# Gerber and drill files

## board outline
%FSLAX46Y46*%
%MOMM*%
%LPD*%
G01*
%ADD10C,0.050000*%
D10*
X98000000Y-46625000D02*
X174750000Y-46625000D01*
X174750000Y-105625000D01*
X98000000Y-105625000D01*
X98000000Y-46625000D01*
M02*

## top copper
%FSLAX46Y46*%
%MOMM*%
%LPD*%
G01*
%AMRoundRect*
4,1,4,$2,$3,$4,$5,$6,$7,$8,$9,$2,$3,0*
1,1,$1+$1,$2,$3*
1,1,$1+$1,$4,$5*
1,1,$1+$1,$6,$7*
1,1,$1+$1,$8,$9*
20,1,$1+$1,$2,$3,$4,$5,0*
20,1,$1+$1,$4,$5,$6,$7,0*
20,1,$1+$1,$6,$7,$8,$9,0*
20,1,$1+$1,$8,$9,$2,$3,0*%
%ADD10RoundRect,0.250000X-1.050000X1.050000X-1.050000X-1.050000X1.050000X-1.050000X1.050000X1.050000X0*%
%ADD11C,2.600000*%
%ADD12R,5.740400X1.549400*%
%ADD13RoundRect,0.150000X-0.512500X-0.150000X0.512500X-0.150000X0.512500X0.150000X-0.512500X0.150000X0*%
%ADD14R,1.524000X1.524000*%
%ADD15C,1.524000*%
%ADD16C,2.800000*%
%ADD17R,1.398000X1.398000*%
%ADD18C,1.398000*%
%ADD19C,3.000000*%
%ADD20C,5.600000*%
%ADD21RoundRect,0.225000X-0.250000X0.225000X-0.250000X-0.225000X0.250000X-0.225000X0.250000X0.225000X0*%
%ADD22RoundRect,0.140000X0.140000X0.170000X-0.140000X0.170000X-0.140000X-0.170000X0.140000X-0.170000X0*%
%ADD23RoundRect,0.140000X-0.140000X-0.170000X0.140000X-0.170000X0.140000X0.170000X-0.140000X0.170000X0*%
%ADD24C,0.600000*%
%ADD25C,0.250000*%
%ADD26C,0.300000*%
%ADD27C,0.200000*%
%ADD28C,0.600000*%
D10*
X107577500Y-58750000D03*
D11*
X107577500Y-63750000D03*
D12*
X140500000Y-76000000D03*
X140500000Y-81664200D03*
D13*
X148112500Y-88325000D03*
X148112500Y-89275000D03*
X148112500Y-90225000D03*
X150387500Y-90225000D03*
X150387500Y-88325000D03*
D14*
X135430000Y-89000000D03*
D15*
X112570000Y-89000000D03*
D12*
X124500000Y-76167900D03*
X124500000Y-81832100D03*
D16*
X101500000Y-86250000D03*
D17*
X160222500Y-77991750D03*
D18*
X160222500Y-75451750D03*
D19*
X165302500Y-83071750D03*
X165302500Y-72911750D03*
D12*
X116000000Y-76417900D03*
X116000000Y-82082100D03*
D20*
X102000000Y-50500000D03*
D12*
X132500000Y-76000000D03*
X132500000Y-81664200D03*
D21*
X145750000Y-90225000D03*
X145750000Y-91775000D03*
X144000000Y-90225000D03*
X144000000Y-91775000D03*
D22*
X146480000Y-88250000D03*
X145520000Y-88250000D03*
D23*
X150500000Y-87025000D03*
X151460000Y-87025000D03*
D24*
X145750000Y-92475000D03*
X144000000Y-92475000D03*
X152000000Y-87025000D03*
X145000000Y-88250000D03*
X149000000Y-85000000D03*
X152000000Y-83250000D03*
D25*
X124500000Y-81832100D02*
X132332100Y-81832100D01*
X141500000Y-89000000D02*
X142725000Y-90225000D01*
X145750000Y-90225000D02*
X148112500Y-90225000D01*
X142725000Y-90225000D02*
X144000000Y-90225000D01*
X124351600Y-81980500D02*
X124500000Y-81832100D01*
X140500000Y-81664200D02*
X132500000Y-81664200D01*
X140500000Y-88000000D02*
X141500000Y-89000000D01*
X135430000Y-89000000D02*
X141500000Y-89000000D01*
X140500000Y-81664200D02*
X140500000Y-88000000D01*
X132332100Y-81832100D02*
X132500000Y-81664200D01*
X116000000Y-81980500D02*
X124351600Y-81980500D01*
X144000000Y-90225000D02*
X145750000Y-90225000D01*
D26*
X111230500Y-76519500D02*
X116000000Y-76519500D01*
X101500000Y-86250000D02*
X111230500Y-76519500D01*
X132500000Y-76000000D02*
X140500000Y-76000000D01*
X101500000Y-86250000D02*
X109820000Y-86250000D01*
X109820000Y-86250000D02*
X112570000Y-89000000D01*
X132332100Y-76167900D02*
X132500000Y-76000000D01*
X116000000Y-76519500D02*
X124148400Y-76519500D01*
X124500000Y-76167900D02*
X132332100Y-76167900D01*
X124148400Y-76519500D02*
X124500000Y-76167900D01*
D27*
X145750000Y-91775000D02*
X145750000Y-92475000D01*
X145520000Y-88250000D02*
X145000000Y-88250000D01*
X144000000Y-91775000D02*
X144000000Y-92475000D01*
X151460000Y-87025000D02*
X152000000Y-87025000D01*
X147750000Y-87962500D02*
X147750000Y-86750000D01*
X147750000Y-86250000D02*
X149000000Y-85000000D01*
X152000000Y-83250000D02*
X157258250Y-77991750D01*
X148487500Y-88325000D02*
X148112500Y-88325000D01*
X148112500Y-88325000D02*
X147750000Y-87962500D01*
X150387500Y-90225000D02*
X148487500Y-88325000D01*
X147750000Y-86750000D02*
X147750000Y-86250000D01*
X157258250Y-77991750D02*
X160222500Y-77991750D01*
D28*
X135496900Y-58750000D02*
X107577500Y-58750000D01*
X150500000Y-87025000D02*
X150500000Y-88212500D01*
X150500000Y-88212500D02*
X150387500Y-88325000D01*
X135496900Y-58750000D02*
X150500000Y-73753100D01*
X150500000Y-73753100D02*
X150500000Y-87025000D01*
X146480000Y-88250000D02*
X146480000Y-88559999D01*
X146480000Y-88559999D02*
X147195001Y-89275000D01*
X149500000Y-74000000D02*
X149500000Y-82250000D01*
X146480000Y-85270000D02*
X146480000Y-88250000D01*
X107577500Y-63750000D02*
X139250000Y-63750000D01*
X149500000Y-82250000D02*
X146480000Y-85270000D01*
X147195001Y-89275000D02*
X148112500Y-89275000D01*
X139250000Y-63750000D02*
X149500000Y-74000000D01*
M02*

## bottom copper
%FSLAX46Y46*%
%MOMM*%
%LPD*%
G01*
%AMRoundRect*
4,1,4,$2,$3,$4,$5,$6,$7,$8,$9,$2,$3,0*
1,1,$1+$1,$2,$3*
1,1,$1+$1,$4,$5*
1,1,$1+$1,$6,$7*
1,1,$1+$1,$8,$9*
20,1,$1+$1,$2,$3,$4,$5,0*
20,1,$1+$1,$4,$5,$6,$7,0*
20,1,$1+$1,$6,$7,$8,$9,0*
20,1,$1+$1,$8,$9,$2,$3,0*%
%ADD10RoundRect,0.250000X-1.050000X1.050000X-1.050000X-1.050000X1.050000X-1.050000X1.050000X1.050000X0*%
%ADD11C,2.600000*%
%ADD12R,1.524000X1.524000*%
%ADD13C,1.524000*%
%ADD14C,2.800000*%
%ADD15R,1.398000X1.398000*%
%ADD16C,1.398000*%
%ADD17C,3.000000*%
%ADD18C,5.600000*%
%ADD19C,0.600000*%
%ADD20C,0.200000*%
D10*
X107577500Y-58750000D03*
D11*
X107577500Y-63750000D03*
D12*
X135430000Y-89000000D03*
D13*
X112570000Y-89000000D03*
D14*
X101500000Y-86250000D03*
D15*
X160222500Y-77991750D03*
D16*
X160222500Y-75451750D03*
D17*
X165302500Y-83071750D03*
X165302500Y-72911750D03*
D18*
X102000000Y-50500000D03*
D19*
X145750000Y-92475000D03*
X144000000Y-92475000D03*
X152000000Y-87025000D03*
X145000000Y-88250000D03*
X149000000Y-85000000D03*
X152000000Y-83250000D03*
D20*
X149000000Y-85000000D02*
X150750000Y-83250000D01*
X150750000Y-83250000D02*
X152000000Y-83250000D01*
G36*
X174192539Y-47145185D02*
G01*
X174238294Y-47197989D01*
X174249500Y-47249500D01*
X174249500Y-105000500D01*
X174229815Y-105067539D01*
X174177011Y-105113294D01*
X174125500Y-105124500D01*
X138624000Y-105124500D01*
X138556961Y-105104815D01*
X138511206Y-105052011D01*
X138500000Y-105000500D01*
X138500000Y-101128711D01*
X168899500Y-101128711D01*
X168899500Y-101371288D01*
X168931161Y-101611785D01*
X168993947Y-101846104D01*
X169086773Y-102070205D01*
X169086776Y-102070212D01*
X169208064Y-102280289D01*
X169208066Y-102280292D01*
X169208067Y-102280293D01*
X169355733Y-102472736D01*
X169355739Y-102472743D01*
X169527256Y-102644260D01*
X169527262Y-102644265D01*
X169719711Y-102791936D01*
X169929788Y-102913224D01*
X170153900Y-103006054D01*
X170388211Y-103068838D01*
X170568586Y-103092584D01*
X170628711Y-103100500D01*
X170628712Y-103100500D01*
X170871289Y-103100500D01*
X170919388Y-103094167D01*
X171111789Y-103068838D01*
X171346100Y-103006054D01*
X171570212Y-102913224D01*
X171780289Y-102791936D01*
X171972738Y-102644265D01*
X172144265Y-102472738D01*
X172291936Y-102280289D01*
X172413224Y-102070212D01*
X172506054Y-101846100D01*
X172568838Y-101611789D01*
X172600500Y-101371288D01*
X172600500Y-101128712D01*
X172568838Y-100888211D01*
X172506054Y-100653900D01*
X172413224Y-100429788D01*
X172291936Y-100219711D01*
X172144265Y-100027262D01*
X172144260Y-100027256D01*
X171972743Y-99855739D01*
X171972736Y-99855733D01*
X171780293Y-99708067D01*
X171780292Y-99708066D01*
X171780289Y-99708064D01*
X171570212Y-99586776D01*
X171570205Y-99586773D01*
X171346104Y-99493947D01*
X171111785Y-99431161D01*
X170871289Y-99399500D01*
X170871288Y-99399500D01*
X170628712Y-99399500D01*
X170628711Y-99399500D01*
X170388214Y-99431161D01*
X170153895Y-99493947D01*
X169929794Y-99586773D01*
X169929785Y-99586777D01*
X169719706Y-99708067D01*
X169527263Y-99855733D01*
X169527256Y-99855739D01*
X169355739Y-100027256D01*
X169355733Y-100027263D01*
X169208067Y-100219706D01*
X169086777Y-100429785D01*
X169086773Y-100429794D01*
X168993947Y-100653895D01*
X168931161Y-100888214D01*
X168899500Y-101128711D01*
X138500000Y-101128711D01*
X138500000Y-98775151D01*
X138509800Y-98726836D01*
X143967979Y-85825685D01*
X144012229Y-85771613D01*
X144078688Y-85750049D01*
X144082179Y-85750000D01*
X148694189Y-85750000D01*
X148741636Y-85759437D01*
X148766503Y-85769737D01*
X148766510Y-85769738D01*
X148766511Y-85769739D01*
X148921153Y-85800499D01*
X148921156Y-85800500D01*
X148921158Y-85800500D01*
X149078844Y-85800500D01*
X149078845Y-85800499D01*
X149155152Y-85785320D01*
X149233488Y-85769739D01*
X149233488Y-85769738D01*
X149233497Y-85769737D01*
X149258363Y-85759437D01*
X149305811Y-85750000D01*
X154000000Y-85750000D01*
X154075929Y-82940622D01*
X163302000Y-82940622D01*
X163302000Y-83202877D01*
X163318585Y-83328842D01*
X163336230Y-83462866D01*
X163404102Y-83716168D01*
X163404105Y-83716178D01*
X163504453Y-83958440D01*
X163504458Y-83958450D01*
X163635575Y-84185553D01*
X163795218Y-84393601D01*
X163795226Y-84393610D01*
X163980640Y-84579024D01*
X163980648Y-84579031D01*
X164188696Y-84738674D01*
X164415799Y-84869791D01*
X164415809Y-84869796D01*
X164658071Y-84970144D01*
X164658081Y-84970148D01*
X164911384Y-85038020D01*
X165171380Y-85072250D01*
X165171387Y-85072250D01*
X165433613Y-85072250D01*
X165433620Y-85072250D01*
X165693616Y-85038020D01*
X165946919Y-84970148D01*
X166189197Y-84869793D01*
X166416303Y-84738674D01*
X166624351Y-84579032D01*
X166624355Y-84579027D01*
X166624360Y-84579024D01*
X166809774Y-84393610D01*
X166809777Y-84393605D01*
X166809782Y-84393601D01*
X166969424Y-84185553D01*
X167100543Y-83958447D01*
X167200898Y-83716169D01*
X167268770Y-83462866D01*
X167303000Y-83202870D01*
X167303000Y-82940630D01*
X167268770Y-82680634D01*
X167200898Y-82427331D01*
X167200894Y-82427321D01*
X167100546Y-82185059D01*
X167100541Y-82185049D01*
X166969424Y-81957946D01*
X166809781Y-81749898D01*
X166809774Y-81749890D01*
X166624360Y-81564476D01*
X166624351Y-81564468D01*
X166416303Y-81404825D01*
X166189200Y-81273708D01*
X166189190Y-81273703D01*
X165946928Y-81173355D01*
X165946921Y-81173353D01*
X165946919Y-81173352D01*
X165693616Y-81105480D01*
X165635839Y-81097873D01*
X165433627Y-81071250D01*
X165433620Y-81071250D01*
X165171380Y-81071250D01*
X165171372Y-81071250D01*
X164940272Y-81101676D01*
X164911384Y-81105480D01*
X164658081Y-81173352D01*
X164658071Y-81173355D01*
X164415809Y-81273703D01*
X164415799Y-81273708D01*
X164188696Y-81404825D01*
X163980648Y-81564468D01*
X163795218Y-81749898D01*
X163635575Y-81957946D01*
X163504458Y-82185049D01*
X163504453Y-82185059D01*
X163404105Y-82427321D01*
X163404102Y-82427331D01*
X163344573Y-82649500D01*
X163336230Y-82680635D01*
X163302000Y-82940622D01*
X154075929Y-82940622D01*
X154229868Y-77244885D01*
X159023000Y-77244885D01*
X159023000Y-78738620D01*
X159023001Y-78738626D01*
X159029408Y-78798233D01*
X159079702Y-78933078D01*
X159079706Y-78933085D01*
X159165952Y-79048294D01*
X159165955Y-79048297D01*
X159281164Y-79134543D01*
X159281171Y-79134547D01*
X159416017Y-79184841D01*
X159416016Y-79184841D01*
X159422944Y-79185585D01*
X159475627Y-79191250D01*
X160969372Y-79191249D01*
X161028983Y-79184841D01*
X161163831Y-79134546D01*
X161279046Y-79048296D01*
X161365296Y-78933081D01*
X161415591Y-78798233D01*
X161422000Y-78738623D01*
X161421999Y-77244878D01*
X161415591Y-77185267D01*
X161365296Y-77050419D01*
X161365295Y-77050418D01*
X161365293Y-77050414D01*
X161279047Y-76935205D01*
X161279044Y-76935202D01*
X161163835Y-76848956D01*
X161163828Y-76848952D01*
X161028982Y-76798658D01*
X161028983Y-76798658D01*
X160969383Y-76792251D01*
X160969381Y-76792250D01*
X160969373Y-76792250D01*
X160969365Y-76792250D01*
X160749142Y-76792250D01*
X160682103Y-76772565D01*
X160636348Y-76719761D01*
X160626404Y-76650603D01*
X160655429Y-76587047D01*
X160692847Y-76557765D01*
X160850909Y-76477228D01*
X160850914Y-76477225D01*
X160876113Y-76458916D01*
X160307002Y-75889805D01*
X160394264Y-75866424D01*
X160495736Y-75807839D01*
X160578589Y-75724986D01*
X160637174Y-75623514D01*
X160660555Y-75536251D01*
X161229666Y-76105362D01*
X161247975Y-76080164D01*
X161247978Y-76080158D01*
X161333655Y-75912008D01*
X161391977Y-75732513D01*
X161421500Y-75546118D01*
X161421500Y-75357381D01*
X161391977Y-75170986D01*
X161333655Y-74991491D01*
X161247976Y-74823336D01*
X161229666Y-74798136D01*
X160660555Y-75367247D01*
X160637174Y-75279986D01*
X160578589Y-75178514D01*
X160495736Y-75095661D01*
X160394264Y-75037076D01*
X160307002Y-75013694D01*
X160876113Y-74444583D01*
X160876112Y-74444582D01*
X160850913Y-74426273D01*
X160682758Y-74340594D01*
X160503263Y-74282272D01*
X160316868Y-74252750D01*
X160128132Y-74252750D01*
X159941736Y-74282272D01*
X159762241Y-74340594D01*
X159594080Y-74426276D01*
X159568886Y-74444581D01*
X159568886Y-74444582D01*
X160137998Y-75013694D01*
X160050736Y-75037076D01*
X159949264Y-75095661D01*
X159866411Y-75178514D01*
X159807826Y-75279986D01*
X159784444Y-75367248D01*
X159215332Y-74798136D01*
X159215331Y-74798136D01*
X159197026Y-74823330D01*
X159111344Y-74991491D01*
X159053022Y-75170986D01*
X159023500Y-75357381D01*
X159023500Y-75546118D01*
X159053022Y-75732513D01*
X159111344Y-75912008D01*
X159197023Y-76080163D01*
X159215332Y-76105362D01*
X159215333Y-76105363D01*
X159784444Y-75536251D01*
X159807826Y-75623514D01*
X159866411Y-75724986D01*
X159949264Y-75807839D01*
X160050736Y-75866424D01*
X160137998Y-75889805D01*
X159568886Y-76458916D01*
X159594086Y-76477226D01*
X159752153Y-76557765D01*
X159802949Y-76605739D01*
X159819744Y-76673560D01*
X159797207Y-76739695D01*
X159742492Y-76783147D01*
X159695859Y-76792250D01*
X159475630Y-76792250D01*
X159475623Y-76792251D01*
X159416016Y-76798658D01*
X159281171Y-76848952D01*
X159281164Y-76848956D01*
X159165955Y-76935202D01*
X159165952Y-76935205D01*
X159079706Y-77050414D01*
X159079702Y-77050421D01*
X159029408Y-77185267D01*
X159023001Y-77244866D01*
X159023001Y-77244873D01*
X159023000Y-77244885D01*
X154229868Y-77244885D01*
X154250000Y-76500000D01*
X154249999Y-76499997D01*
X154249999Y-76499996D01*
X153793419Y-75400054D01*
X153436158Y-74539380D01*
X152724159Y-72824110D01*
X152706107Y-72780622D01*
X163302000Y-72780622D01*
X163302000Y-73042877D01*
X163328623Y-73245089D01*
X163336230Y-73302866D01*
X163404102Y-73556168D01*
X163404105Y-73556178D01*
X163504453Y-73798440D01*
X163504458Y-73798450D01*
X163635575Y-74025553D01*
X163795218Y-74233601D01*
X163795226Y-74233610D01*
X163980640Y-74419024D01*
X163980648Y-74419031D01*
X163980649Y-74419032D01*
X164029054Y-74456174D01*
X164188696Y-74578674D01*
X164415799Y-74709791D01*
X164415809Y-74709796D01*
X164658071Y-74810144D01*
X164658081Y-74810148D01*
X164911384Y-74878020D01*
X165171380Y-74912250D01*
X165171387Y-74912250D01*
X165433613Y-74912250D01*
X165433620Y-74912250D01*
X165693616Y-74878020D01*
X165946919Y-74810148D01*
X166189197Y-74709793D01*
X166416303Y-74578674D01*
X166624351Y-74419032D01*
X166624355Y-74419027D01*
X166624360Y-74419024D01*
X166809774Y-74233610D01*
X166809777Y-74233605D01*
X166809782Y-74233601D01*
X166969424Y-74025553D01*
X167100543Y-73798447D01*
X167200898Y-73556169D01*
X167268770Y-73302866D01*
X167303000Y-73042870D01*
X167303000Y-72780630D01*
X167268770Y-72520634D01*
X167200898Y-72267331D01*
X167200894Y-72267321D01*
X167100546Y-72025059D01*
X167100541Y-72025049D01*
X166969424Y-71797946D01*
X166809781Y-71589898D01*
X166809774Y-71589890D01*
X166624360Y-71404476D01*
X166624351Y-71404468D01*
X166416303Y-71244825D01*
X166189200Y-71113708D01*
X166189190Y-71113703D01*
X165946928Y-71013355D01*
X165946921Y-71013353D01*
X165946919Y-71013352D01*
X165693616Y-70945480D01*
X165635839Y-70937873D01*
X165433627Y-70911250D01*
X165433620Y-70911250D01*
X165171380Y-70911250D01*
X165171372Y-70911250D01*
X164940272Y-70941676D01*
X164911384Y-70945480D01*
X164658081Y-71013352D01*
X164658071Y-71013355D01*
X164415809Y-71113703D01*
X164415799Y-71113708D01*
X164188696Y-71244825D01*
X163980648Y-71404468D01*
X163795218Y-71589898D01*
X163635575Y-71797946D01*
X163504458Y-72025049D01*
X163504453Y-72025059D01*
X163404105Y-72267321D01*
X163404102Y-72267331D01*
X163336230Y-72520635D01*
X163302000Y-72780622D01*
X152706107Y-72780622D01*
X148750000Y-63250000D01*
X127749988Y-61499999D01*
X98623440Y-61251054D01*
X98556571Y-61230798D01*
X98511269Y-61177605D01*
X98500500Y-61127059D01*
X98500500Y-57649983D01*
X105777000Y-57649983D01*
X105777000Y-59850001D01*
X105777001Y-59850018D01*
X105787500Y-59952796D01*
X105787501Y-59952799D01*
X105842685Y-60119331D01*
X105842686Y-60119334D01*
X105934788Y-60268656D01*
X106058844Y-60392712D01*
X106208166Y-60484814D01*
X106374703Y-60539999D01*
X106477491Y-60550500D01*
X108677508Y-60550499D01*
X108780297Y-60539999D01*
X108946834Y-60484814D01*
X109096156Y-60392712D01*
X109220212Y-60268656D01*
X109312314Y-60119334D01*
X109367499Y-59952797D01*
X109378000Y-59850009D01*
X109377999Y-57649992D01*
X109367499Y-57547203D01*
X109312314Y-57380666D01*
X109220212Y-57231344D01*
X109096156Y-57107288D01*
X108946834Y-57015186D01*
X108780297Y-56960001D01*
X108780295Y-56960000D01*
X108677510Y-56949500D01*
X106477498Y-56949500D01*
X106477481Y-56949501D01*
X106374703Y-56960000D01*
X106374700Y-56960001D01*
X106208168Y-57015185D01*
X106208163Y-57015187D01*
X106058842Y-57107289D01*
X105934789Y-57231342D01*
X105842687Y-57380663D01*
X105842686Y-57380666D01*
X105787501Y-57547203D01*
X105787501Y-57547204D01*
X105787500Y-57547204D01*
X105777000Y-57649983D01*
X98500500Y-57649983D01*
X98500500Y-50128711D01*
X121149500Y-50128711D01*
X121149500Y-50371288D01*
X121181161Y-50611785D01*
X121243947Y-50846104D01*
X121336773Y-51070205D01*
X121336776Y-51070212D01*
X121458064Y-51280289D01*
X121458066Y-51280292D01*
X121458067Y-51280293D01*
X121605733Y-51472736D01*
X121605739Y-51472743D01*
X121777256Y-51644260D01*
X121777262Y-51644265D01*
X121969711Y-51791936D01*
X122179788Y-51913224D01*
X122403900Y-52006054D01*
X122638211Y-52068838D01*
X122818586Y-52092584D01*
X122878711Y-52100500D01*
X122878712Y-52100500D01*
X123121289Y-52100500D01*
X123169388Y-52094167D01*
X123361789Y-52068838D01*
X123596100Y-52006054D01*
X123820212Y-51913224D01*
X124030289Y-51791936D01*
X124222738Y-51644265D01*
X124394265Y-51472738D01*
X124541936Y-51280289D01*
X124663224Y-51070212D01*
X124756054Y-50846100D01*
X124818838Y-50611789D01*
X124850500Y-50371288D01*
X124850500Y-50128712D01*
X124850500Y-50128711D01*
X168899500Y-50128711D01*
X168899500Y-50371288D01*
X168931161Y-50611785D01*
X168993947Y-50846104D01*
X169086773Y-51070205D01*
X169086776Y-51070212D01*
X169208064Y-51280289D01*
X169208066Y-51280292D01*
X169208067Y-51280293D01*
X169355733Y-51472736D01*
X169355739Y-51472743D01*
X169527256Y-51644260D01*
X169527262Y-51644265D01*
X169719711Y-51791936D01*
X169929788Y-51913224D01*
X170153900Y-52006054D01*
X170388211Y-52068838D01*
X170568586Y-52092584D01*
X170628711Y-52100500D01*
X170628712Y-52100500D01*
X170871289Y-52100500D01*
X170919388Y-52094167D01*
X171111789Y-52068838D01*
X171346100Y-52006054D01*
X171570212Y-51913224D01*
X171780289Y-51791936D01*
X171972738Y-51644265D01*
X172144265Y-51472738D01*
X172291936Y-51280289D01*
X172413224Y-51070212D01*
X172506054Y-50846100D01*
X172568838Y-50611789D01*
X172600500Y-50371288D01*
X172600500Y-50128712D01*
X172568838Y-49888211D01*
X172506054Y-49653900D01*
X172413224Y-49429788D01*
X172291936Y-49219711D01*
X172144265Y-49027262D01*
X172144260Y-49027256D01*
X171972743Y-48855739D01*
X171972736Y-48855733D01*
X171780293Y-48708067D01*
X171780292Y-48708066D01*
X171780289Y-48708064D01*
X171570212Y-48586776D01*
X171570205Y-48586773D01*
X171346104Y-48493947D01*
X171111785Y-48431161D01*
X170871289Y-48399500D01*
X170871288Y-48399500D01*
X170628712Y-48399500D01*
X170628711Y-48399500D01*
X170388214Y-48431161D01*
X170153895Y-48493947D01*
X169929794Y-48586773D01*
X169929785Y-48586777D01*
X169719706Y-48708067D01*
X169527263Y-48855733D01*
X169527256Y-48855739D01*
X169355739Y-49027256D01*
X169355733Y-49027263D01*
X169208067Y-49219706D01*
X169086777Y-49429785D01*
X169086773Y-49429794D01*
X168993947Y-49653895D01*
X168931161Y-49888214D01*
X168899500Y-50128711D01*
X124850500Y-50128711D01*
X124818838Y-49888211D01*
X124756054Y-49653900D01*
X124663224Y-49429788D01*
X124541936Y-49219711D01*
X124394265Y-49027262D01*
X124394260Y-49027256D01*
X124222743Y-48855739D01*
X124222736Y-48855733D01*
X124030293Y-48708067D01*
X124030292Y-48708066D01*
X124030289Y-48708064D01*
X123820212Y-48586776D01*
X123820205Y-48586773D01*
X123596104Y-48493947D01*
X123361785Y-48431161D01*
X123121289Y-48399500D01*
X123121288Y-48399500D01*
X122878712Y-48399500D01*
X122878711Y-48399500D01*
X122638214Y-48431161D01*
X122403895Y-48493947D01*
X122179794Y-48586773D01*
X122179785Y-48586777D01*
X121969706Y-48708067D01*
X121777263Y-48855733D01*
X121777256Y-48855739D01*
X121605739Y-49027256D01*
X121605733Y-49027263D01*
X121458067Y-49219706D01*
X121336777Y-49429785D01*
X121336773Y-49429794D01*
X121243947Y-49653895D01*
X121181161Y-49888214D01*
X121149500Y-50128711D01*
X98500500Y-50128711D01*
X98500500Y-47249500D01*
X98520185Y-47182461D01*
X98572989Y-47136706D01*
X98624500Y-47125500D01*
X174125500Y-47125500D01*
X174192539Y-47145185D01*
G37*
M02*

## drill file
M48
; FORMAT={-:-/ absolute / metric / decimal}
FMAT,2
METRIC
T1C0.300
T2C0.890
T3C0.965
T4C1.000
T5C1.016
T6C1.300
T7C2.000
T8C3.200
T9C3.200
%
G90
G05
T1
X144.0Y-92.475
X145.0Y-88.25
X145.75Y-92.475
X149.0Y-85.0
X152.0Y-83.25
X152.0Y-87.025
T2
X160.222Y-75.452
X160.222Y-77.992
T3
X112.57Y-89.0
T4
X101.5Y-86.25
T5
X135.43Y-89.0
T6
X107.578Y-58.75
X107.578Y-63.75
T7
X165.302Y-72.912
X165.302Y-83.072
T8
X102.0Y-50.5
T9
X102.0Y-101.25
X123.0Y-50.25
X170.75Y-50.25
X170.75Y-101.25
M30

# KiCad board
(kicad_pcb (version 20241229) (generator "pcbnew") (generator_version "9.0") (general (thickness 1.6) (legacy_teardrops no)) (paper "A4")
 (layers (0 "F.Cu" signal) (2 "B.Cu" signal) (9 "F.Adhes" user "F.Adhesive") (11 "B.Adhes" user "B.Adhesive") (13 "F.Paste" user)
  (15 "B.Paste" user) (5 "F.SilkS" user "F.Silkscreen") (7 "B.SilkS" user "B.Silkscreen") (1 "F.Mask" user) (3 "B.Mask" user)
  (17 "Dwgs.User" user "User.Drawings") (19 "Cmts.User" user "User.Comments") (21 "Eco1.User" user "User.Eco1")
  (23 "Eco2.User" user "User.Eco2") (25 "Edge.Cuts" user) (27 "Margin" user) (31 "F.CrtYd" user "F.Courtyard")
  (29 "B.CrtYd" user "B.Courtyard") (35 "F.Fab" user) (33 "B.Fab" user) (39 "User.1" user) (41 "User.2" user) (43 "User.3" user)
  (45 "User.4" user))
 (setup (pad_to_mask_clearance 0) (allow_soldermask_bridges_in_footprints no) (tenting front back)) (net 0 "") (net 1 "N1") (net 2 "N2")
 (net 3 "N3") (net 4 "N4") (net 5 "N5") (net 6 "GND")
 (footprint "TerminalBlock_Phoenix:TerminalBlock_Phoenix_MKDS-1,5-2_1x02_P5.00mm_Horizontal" (layer "F.Cu") (at 107.5775 58.75 -90)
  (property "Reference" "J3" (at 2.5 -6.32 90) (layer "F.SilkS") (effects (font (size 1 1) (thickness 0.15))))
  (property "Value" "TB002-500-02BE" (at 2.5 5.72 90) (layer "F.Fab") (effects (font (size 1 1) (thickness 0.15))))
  (pad "1" thru_hole roundrect (at 0 0 270) (size 2.6 2.6) (drill 1.3) (layers "*.Cu" "*.Mask") (remove_unused_layers no)
   (roundrect_rratio 0.096154) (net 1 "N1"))
  (pad "2" thru_hole circle (at 5 0 270) (size 2.6 2.6) (drill 1.3) (layers "*.Cu" "*.Mask") (remove_unused_layers no) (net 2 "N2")))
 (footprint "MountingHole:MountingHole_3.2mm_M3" (layer "F.Cu") (at 123 50.25)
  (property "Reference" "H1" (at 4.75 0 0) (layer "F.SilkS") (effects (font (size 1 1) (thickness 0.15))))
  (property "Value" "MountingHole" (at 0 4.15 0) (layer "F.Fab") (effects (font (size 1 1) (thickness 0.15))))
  (pad "" np_thru_hole circle (at 0 0) (size 3.2 3.2) (drill 3.2) (layers "*.Cu" "*.Mask")))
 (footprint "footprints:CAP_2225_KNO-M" (layer "F.Cu") (at 140.5 78.8321 -90)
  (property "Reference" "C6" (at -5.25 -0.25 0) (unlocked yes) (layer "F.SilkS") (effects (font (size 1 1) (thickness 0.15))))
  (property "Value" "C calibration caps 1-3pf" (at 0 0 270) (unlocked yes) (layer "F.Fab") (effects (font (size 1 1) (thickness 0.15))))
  (pad "1" smd rect (at -2.8321 0 270) (size 1.5494 5.7404) (layers "F.Cu" "F.Mask" "F.Paste") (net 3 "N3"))
  (pad "2" smd rect (at 2.8321 0 270) (size 1.5494 5.7404) (layers "F.Cu" "F.Mask" "F.Paste") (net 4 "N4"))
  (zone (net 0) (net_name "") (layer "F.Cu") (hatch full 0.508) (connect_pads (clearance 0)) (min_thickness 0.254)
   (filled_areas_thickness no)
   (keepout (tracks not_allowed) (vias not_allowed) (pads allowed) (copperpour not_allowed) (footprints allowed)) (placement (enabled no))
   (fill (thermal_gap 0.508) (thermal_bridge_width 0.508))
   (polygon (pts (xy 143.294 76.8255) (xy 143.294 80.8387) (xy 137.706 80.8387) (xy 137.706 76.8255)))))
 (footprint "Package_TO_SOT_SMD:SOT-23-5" (layer "F.Cu") (at 149.25 89.275)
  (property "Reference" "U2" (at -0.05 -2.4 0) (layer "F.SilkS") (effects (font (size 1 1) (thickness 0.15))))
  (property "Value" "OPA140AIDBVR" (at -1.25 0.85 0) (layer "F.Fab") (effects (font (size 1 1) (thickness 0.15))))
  (pad "1" smd roundrect (at -1.1375 -0.95) (size 1.325 0.6) (layers "F.Cu" "F.Mask" "F.Paste") (roundrect_rratio 0.25) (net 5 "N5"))
  (pad "2" smd roundrect (at -1.1375 0) (size 1.325 0.6) (layers "F.Cu" "F.Mask" "F.Paste") (roundrect_rratio 0.25) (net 2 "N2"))
  (pad "3" smd roundrect (at -1.1375 0.95) (size 1.325 0.6) (layers "F.Cu" "F.Mask" "F.Paste") (roundrect_rratio 0.25) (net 4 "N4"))
  (pad "4" smd roundrect (at 1.1375 0.95) (size 1.325 0.6) (layers "F.Cu" "F.Mask" "F.Paste") (roundrect_rratio 0.25) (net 5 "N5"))
  (pad "5" smd roundrect (at 1.1375 -0.95) (size 1.325 0.6) (layers "F.Cu" "F.Mask" "F.Paste") (roundrect_rratio 0.25) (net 1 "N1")))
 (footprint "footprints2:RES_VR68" (layer "F.Cu") (at 112.57 89 180)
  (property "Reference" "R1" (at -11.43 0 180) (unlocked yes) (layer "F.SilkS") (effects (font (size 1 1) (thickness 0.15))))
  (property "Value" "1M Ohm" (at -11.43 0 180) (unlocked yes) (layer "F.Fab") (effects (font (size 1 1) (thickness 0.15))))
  (pad "1" thru_hole rect (at -22.86 0 180) (size 1.524 1.524) (drill 1.016) (layers "*.Cu" "*.Mask") (remove_unused_layers no) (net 4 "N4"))
  (pad "2" thru_hole circle (at 0 0 180) (size 1.524 1.524) (drill 0.9652) (layers "*.Cu" "*.Mask") (remove_unused_layers no) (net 3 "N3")))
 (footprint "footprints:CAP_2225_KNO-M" (layer "F.Cu") (at 124.5 79 -90)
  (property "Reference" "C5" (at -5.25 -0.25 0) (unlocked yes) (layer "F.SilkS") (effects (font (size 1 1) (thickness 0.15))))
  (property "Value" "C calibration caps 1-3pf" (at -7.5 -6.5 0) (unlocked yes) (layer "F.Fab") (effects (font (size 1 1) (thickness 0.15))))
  (pad "1" smd rect (at -2.8321 0 270) (size 1.5494 5.7404) (layers "F.Cu" "F.Mask" "F.Paste") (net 3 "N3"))
  (pad "2" smd rect (at 2.8321 0 270) (size 1.5494 5.7404) (layers "F.Cu" "F.Mask" "F.Paste") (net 4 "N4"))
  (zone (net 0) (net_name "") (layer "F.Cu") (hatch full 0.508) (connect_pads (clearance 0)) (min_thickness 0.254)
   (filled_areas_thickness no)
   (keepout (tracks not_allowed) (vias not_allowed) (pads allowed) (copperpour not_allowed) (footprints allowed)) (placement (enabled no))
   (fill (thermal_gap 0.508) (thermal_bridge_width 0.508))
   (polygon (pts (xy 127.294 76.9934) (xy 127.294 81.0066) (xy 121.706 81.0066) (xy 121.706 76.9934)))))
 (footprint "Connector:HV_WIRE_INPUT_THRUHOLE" (layer "F.Cu") (at 101.5 89.25)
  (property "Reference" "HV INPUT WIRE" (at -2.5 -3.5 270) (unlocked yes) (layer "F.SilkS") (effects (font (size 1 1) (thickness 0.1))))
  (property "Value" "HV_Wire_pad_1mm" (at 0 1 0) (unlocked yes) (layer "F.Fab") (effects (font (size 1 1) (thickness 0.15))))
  (pad "1" thru_hole circle (at 0 -3) (size 2.8 2.8) (drill 1) (layers "*.Cu" "*.Mask") (remove_unused_layers no) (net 3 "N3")))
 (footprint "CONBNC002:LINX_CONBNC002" (layer "F.Cu") (at 165.3025 77.99175 90)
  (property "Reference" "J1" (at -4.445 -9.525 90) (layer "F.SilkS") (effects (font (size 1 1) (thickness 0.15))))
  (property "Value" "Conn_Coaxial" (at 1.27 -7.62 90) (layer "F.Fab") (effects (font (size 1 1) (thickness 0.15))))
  (pad "1" thru_hole rect (at 0 -5.08 90) (size 1.398 1.398) (drill 0.89) (layers "*.Cu" "*.Mask") (remove_unused_layers no) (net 5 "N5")
   (solder_mask_margin 0.102))
  (pad "2" thru_hole circle (at 2.54 -5.08 90) (size 1.398 1.398) (drill 0.89) (layers "*.Cu" "*.Mask") (remove_unused_layers no)
   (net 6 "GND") (solder_mask_margin 0.102))
  (pad "S1" thru_hole circle (at -5.08 0 90) (size 3 3) (drill 2) (layers "*.Cu" "*.Mask") (remove_unused_layers no)
   (solder_mask_margin 0.102))
  (pad "S2" thru_hole circle (at 5.08 0 90) (size 3 3) (drill 2) (layers "*.Cu" "*.Mask") (remove_unused_layers no)
   (solder_mask_margin 0.102)))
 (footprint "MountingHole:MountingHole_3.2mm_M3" (layer "F.Cu") (at 170.75 101.25)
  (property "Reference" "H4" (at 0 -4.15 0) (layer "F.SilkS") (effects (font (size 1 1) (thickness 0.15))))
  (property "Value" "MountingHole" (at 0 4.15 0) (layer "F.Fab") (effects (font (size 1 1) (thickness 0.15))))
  (pad "" np_thru_hole circle (at 0 0) (size 3.2 3.2) (drill 3.2) (layers "*.Cu" "*.Mask")))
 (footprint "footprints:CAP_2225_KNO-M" (layer "F.Cu") (at 116 79.25 -90)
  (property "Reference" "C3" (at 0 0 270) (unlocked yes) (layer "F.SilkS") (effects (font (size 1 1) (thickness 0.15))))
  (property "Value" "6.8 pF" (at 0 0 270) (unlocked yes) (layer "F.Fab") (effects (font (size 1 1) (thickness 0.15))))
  (pad "1" smd rect (at -2.8321 0 270) (size 1.5494 5.7404) (layers "F.Cu" "F.Mask" "F.Paste") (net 3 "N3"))
  (pad "2" smd rect (at 2.8321 0 270) (size 1.5494 5.7404) (layers "F.Cu" "F.Mask" "F.Paste") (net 4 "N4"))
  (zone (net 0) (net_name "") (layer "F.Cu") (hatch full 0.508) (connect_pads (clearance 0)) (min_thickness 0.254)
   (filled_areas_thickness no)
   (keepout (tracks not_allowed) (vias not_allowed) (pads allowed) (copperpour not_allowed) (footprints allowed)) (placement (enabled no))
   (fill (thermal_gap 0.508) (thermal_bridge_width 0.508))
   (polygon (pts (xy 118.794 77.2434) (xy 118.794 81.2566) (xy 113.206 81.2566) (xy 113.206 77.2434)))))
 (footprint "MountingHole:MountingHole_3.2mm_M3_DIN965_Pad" (layer "F.Cu") (at 102 50.5)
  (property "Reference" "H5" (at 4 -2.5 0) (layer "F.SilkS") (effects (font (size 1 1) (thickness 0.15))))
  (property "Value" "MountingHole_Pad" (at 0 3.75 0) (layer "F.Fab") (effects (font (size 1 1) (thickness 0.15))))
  (pad "1" thru_hole circle (at 0 0) (size 5.6 5.6) (drill 3.2) (layers "*.Cu" "*.Mask") (remove_unused_layers no) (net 6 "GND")
   (zone_connect 2)))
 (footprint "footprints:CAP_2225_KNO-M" (layer "F.Cu") (at 132.5 78.8321 -90)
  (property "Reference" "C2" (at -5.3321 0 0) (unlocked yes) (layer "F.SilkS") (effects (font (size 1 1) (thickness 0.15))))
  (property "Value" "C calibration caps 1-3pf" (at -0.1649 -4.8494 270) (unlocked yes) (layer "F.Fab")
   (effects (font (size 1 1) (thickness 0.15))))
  (pad "1" smd rect (at -2.8321 0 270) (size 1.5494 5.7404) (layers "F.Cu" "F.Mask" "F.Paste") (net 3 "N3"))
  (pad "2" smd rect (at 2.8321 0 270) (size 1.5494 5.7404) (layers "F.Cu" "F.Mask" "F.Paste") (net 4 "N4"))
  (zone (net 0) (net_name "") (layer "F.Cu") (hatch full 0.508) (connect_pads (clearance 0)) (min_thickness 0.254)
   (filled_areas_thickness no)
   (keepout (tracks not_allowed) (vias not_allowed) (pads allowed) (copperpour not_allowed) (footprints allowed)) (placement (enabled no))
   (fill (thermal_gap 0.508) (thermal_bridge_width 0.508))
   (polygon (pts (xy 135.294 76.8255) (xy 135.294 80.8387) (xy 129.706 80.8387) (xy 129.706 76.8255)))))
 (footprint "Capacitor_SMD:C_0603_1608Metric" (layer "F.Cu") (at 145.75 91 -90)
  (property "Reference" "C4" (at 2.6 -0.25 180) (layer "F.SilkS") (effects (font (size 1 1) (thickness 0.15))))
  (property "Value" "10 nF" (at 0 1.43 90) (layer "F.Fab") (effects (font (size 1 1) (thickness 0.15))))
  (pad "1" smd roundrect (at -0.775 0 270) (size 0.9 0.95) (layers "F.Cu" "F.Mask" "F.Paste") (roundrect_rratio 0.25) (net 4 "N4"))
  (pad "2" smd roundrect (at 0.775 0 270) (size 0.9 0.95) (layers "F.Cu" "F.Mask" "F.Paste") (roundrect_rratio 0.25) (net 6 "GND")))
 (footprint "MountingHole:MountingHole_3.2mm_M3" (layer "F.Cu") (at 102 101.25)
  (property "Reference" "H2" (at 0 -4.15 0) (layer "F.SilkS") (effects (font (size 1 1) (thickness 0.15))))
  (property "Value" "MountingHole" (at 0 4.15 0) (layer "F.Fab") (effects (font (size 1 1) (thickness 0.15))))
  (pad "" np_thru_hole circle (at 0 0) (size 3.2 3.2) (drill 3.2) (layers "*.Cu" "*.Mask")))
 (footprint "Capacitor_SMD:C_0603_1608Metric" (layer "F.Cu") (at 144 91 -90)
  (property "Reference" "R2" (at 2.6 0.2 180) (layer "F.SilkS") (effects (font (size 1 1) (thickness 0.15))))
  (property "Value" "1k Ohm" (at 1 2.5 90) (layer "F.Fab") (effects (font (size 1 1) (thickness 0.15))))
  (pad "1" smd roundrect (at -0.775 0 270) (size 0.9 0.95) (layers "F.Cu" "F.Mask" "F.Paste") (roundrect_rratio 0.25) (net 4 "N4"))
  (pad "2" smd roundrect (at 0.775 0 270) (size 0.9 0.95) (layers "F.Cu" "F.Mask" "F.Paste") (roundrect_rratio 0.25) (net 6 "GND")))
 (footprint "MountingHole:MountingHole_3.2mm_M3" (layer "F.Cu") (at 170.75 50.25)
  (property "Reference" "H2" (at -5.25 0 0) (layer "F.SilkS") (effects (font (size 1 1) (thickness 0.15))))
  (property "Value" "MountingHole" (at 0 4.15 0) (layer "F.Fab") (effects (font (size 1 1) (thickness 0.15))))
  (pad "" np_thru_hole circle (at 0 0) (size 3.2 3.2) (drill 3.2) (layers "*.Cu" "*.Mask")))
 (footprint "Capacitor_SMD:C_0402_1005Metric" (layer "F.Cu") (at 146 88.25 180)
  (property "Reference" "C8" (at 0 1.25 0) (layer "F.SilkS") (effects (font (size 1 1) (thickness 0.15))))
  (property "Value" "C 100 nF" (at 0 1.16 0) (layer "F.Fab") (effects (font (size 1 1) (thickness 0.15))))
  (pad "1" smd roundrect (at -0.48 0 180) (size 0.56 0.62) (layers "F.Cu" "F.Mask" "F.Paste") (roundrect_rratio 0.25) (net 2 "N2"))
  (pad "2" smd roundrect (at 0.48 0 180) (size 0.56 0.62) (layers "F.Cu" "F.Mask" "F.Paste") (roundrect_rratio 0.25) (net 6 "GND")))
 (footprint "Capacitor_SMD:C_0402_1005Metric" (layer "F.Cu") (at 150.98 87.025)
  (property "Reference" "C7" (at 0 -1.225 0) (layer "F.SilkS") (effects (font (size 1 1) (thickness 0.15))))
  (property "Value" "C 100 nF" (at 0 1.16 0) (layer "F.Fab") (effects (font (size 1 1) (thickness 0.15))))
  (pad "1" smd roundrect (at -0.48 0) (size 0.56 0.62) (layers "F.Cu" "F.Mask" "F.Paste") (roundrect_rratio 0.25) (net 1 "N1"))
  (pad "2" smd roundrect (at 0.48 0) (size 0.56 0.62) (layers "F.Cu" "F.Mask" "F.Paste") (roundrect_rratio 0.25) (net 6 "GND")))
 (gr_rect (start 98 46.625) (end 174.75 105.625) (stroke (width 0.05) (type default)) (fill no) (layer "Edge.Cuts"))
 (segment (start 124.5 81.8321) (end 132.3321 81.8321) (width 0.25) (layer "F.Cu") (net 4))
 (segment (start 141.5 89) (end 142.725 90.225) (width 0.25) (layer "F.Cu") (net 4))
 (segment (start 145.75 90.225) (end 148.1125 90.225) (width 0.25) (layer "F.Cu") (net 4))
 (segment (start 142.725 90.225) (end 144 90.225) (width 0.25) (layer "F.Cu") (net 4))
 (segment (start 124.3516 81.9805) (end 124.5 81.8321) (width 0.25) (layer "F.Cu") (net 4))
 (segment (start 140.5 81.6642) (end 132.5 81.6642) (width 0.25) (layer "F.Cu") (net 4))
 (segment (start 140.5 88) (end 141.5 89) (width 0.25) (layer "F.Cu") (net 4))
 (segment (start 135.43 89) (end 141.5 89) (width 0.25) (layer "F.Cu") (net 4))
 (segment (start 140.5 81.6642) (end 140.5 88) (width 0.25) (layer "F.Cu") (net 4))
 (segment (start 132.3321 81.8321) (end 132.5 81.6642) (width 0.25) (layer "F.Cu") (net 4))
 (segment (start 116 81.9805) (end 124.3516 81.9805) (width 0.25) (layer "F.Cu") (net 4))
 (segment (start 144 90.225) (end 145.75 90.225) (width 0.25) (layer "F.Cu") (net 4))
 (segment (start 111.2305 76.5195) (end 116 76.5195) (width 0.3) (layer "F.Cu") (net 3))
 (segment (start 101.5 86.25) (end 111.2305 76.5195) (width 0.3) (layer "F.Cu") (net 3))
 (segment (start 132.5 76) (end 140.5 76) (width 0.3) (layer "F.Cu") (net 3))
 (segment (start 101.5 86.25) (end 109.82 86.25) (width 0.3) (layer "F.Cu") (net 3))
 (segment (start 109.82 86.25) (end 112.57 89) (width 0.3) (layer "F.Cu") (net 3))
 (segment (start 132.3321 76.1679) (end 132.5 76) (width 0.3) (layer "F.Cu") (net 3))
 (segment (start 116 76.5195) (end 124.1484 76.5195) (width 0.3) (layer "F.Cu") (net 3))
 (segment (start 124.5 76.1679) (end 132.3321 76.1679) (width 0.3) (layer "F.Cu") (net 3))
 (segment (start 124.1484 76.5195) (end 124.5 76.1679) (width 0.3) (layer "F.Cu") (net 3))
 (segment (start 145.75 91.775) (end 145.75 92.475) (width 0.2) (layer "F.Cu") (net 6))
 (segment (start 145.52 88.25) (end 145 88.25) (width 0.2) (layer "F.Cu") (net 6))
 (segment (start 144 91.775) (end 144 92.475) (width 0.2) (layer "F.Cu") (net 6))
 (segment (start 151.46 87.025) (end 152 87.025) (width 0.2) (layer "F.Cu") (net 6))
 (via (at 145.75 92.475) (size 0.6) (drill 0.3) (layers "F.Cu" "B.Cu") (free yes) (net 6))
 (via (at 144 92.475) (size 0.6) (drill 0.3) (layers "F.Cu" "B.Cu") (free yes) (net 6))
 (via (at 152 87.025) (size 0.6) (drill 0.3) (layers "F.Cu" "B.Cu") (free yes) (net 6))
 (via (at 145 88.25) (size 0.6) (drill 0.3) (layers "F.Cu" "B.Cu") (free yes) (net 6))
 (segment (start 147.75 87.9625) (end 147.75 86.75) (width 0.2) (layer "F.Cu") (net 5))
 (segment (start 147.75 86.25) (end 149 85) (width 0.2) (layer "F.Cu") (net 5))
 (segment (start 152 83.25) (end 157.25825 77.99175) (width 0.2) (layer "F.Cu") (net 5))
 (segment (start 148.4875 88.325) (end 148.1125 88.325) (width 0.2) (layer "F.Cu") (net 5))
 (segment (start 148.1125 88.325) (end 147.75 87.9625) (width 0.2) (layer "F.Cu") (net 5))
 (segment (start 150.3875 90.225) (end 148.4875 88.325) (width 0.2) (layer "F.Cu") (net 5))
 (segment (start 147.75 86.75) (end 147.75 86.25) (width 0.2) (layer "F.Cu") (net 5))
 (segment (start 157.25825 77.99175) (end 160.2225 77.99175) (width 0.2) (layer "F.Cu") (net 5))
 (via (at 149 85) (size 0.6) (drill 0.3) (layers "F.Cu" "B.Cu") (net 5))
 (via (at 152 83.25) (size 0.6) (drill 0.3) (layers "F.Cu" "B.Cu") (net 5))
 (segment (start 149 85) (end 150.75 83.25) (width 0.2) (layer "B.Cu") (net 5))
 (segment (start 150.75 83.25) (end 152 83.25) (width 0.2) (layer "B.Cu") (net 5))
 (segment (start 135.4969 58.75) (end 107.5775 58.75) (width 0.6) (layer "F.Cu") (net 1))
 (segment (start 150.5 87.025) (end 150.5 88.2125) (width 0.6) (layer "F.Cu") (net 1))
 (segment (start 150.5 88.2125) (end 150.3875 88.325) (width 0.6) (layer "F.Cu") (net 1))
 (segment (start 135.4969 58.75) (end 150.5 73.7531) (width 0.6) (layer "F.Cu") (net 1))
 (segment (start 150.5 73.7531) (end 150.5 87.025) (width 0.6) (layer "F.Cu") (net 1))
 (segment (start 146.48 88.25) (end 146.48 88.559999) (width 0.6) (layer "F.Cu") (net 2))
 (segment (start 146.48 88.559999) (end 147.195001 89.275) (width 0.6) (layer "F.Cu") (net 2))
 (segment (start 149.5 74) (end 149.5 82.25) (width 0.6) (layer "F.Cu") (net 2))
 (segment (start 146.48 85.27) (end 146.48 88.25) (width 0.6) (layer "F.Cu") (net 2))
 (segment (start 107.5775 63.75) (end 139.25 63.75) (width 0.6) (layer "F.Cu") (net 2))
 (segment (start 149.5 82.25) (end 146.48 85.27) (width 0.6) (layer "F.Cu") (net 2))
 (segment (start 147.195001 89.275) (end 148.1125 89.275) (width 0.6) (layer "F.Cu") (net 2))
 (segment (start 139.25 63.75) (end 149.5 74) (width 0.6) (layer "F.Cu") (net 2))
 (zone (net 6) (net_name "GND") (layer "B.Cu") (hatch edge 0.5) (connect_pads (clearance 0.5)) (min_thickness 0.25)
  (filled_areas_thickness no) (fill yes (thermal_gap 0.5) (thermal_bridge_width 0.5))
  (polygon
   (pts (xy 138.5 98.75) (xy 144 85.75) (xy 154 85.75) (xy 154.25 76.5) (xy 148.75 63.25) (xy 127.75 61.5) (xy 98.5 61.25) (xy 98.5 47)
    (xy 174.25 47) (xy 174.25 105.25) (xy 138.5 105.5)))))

